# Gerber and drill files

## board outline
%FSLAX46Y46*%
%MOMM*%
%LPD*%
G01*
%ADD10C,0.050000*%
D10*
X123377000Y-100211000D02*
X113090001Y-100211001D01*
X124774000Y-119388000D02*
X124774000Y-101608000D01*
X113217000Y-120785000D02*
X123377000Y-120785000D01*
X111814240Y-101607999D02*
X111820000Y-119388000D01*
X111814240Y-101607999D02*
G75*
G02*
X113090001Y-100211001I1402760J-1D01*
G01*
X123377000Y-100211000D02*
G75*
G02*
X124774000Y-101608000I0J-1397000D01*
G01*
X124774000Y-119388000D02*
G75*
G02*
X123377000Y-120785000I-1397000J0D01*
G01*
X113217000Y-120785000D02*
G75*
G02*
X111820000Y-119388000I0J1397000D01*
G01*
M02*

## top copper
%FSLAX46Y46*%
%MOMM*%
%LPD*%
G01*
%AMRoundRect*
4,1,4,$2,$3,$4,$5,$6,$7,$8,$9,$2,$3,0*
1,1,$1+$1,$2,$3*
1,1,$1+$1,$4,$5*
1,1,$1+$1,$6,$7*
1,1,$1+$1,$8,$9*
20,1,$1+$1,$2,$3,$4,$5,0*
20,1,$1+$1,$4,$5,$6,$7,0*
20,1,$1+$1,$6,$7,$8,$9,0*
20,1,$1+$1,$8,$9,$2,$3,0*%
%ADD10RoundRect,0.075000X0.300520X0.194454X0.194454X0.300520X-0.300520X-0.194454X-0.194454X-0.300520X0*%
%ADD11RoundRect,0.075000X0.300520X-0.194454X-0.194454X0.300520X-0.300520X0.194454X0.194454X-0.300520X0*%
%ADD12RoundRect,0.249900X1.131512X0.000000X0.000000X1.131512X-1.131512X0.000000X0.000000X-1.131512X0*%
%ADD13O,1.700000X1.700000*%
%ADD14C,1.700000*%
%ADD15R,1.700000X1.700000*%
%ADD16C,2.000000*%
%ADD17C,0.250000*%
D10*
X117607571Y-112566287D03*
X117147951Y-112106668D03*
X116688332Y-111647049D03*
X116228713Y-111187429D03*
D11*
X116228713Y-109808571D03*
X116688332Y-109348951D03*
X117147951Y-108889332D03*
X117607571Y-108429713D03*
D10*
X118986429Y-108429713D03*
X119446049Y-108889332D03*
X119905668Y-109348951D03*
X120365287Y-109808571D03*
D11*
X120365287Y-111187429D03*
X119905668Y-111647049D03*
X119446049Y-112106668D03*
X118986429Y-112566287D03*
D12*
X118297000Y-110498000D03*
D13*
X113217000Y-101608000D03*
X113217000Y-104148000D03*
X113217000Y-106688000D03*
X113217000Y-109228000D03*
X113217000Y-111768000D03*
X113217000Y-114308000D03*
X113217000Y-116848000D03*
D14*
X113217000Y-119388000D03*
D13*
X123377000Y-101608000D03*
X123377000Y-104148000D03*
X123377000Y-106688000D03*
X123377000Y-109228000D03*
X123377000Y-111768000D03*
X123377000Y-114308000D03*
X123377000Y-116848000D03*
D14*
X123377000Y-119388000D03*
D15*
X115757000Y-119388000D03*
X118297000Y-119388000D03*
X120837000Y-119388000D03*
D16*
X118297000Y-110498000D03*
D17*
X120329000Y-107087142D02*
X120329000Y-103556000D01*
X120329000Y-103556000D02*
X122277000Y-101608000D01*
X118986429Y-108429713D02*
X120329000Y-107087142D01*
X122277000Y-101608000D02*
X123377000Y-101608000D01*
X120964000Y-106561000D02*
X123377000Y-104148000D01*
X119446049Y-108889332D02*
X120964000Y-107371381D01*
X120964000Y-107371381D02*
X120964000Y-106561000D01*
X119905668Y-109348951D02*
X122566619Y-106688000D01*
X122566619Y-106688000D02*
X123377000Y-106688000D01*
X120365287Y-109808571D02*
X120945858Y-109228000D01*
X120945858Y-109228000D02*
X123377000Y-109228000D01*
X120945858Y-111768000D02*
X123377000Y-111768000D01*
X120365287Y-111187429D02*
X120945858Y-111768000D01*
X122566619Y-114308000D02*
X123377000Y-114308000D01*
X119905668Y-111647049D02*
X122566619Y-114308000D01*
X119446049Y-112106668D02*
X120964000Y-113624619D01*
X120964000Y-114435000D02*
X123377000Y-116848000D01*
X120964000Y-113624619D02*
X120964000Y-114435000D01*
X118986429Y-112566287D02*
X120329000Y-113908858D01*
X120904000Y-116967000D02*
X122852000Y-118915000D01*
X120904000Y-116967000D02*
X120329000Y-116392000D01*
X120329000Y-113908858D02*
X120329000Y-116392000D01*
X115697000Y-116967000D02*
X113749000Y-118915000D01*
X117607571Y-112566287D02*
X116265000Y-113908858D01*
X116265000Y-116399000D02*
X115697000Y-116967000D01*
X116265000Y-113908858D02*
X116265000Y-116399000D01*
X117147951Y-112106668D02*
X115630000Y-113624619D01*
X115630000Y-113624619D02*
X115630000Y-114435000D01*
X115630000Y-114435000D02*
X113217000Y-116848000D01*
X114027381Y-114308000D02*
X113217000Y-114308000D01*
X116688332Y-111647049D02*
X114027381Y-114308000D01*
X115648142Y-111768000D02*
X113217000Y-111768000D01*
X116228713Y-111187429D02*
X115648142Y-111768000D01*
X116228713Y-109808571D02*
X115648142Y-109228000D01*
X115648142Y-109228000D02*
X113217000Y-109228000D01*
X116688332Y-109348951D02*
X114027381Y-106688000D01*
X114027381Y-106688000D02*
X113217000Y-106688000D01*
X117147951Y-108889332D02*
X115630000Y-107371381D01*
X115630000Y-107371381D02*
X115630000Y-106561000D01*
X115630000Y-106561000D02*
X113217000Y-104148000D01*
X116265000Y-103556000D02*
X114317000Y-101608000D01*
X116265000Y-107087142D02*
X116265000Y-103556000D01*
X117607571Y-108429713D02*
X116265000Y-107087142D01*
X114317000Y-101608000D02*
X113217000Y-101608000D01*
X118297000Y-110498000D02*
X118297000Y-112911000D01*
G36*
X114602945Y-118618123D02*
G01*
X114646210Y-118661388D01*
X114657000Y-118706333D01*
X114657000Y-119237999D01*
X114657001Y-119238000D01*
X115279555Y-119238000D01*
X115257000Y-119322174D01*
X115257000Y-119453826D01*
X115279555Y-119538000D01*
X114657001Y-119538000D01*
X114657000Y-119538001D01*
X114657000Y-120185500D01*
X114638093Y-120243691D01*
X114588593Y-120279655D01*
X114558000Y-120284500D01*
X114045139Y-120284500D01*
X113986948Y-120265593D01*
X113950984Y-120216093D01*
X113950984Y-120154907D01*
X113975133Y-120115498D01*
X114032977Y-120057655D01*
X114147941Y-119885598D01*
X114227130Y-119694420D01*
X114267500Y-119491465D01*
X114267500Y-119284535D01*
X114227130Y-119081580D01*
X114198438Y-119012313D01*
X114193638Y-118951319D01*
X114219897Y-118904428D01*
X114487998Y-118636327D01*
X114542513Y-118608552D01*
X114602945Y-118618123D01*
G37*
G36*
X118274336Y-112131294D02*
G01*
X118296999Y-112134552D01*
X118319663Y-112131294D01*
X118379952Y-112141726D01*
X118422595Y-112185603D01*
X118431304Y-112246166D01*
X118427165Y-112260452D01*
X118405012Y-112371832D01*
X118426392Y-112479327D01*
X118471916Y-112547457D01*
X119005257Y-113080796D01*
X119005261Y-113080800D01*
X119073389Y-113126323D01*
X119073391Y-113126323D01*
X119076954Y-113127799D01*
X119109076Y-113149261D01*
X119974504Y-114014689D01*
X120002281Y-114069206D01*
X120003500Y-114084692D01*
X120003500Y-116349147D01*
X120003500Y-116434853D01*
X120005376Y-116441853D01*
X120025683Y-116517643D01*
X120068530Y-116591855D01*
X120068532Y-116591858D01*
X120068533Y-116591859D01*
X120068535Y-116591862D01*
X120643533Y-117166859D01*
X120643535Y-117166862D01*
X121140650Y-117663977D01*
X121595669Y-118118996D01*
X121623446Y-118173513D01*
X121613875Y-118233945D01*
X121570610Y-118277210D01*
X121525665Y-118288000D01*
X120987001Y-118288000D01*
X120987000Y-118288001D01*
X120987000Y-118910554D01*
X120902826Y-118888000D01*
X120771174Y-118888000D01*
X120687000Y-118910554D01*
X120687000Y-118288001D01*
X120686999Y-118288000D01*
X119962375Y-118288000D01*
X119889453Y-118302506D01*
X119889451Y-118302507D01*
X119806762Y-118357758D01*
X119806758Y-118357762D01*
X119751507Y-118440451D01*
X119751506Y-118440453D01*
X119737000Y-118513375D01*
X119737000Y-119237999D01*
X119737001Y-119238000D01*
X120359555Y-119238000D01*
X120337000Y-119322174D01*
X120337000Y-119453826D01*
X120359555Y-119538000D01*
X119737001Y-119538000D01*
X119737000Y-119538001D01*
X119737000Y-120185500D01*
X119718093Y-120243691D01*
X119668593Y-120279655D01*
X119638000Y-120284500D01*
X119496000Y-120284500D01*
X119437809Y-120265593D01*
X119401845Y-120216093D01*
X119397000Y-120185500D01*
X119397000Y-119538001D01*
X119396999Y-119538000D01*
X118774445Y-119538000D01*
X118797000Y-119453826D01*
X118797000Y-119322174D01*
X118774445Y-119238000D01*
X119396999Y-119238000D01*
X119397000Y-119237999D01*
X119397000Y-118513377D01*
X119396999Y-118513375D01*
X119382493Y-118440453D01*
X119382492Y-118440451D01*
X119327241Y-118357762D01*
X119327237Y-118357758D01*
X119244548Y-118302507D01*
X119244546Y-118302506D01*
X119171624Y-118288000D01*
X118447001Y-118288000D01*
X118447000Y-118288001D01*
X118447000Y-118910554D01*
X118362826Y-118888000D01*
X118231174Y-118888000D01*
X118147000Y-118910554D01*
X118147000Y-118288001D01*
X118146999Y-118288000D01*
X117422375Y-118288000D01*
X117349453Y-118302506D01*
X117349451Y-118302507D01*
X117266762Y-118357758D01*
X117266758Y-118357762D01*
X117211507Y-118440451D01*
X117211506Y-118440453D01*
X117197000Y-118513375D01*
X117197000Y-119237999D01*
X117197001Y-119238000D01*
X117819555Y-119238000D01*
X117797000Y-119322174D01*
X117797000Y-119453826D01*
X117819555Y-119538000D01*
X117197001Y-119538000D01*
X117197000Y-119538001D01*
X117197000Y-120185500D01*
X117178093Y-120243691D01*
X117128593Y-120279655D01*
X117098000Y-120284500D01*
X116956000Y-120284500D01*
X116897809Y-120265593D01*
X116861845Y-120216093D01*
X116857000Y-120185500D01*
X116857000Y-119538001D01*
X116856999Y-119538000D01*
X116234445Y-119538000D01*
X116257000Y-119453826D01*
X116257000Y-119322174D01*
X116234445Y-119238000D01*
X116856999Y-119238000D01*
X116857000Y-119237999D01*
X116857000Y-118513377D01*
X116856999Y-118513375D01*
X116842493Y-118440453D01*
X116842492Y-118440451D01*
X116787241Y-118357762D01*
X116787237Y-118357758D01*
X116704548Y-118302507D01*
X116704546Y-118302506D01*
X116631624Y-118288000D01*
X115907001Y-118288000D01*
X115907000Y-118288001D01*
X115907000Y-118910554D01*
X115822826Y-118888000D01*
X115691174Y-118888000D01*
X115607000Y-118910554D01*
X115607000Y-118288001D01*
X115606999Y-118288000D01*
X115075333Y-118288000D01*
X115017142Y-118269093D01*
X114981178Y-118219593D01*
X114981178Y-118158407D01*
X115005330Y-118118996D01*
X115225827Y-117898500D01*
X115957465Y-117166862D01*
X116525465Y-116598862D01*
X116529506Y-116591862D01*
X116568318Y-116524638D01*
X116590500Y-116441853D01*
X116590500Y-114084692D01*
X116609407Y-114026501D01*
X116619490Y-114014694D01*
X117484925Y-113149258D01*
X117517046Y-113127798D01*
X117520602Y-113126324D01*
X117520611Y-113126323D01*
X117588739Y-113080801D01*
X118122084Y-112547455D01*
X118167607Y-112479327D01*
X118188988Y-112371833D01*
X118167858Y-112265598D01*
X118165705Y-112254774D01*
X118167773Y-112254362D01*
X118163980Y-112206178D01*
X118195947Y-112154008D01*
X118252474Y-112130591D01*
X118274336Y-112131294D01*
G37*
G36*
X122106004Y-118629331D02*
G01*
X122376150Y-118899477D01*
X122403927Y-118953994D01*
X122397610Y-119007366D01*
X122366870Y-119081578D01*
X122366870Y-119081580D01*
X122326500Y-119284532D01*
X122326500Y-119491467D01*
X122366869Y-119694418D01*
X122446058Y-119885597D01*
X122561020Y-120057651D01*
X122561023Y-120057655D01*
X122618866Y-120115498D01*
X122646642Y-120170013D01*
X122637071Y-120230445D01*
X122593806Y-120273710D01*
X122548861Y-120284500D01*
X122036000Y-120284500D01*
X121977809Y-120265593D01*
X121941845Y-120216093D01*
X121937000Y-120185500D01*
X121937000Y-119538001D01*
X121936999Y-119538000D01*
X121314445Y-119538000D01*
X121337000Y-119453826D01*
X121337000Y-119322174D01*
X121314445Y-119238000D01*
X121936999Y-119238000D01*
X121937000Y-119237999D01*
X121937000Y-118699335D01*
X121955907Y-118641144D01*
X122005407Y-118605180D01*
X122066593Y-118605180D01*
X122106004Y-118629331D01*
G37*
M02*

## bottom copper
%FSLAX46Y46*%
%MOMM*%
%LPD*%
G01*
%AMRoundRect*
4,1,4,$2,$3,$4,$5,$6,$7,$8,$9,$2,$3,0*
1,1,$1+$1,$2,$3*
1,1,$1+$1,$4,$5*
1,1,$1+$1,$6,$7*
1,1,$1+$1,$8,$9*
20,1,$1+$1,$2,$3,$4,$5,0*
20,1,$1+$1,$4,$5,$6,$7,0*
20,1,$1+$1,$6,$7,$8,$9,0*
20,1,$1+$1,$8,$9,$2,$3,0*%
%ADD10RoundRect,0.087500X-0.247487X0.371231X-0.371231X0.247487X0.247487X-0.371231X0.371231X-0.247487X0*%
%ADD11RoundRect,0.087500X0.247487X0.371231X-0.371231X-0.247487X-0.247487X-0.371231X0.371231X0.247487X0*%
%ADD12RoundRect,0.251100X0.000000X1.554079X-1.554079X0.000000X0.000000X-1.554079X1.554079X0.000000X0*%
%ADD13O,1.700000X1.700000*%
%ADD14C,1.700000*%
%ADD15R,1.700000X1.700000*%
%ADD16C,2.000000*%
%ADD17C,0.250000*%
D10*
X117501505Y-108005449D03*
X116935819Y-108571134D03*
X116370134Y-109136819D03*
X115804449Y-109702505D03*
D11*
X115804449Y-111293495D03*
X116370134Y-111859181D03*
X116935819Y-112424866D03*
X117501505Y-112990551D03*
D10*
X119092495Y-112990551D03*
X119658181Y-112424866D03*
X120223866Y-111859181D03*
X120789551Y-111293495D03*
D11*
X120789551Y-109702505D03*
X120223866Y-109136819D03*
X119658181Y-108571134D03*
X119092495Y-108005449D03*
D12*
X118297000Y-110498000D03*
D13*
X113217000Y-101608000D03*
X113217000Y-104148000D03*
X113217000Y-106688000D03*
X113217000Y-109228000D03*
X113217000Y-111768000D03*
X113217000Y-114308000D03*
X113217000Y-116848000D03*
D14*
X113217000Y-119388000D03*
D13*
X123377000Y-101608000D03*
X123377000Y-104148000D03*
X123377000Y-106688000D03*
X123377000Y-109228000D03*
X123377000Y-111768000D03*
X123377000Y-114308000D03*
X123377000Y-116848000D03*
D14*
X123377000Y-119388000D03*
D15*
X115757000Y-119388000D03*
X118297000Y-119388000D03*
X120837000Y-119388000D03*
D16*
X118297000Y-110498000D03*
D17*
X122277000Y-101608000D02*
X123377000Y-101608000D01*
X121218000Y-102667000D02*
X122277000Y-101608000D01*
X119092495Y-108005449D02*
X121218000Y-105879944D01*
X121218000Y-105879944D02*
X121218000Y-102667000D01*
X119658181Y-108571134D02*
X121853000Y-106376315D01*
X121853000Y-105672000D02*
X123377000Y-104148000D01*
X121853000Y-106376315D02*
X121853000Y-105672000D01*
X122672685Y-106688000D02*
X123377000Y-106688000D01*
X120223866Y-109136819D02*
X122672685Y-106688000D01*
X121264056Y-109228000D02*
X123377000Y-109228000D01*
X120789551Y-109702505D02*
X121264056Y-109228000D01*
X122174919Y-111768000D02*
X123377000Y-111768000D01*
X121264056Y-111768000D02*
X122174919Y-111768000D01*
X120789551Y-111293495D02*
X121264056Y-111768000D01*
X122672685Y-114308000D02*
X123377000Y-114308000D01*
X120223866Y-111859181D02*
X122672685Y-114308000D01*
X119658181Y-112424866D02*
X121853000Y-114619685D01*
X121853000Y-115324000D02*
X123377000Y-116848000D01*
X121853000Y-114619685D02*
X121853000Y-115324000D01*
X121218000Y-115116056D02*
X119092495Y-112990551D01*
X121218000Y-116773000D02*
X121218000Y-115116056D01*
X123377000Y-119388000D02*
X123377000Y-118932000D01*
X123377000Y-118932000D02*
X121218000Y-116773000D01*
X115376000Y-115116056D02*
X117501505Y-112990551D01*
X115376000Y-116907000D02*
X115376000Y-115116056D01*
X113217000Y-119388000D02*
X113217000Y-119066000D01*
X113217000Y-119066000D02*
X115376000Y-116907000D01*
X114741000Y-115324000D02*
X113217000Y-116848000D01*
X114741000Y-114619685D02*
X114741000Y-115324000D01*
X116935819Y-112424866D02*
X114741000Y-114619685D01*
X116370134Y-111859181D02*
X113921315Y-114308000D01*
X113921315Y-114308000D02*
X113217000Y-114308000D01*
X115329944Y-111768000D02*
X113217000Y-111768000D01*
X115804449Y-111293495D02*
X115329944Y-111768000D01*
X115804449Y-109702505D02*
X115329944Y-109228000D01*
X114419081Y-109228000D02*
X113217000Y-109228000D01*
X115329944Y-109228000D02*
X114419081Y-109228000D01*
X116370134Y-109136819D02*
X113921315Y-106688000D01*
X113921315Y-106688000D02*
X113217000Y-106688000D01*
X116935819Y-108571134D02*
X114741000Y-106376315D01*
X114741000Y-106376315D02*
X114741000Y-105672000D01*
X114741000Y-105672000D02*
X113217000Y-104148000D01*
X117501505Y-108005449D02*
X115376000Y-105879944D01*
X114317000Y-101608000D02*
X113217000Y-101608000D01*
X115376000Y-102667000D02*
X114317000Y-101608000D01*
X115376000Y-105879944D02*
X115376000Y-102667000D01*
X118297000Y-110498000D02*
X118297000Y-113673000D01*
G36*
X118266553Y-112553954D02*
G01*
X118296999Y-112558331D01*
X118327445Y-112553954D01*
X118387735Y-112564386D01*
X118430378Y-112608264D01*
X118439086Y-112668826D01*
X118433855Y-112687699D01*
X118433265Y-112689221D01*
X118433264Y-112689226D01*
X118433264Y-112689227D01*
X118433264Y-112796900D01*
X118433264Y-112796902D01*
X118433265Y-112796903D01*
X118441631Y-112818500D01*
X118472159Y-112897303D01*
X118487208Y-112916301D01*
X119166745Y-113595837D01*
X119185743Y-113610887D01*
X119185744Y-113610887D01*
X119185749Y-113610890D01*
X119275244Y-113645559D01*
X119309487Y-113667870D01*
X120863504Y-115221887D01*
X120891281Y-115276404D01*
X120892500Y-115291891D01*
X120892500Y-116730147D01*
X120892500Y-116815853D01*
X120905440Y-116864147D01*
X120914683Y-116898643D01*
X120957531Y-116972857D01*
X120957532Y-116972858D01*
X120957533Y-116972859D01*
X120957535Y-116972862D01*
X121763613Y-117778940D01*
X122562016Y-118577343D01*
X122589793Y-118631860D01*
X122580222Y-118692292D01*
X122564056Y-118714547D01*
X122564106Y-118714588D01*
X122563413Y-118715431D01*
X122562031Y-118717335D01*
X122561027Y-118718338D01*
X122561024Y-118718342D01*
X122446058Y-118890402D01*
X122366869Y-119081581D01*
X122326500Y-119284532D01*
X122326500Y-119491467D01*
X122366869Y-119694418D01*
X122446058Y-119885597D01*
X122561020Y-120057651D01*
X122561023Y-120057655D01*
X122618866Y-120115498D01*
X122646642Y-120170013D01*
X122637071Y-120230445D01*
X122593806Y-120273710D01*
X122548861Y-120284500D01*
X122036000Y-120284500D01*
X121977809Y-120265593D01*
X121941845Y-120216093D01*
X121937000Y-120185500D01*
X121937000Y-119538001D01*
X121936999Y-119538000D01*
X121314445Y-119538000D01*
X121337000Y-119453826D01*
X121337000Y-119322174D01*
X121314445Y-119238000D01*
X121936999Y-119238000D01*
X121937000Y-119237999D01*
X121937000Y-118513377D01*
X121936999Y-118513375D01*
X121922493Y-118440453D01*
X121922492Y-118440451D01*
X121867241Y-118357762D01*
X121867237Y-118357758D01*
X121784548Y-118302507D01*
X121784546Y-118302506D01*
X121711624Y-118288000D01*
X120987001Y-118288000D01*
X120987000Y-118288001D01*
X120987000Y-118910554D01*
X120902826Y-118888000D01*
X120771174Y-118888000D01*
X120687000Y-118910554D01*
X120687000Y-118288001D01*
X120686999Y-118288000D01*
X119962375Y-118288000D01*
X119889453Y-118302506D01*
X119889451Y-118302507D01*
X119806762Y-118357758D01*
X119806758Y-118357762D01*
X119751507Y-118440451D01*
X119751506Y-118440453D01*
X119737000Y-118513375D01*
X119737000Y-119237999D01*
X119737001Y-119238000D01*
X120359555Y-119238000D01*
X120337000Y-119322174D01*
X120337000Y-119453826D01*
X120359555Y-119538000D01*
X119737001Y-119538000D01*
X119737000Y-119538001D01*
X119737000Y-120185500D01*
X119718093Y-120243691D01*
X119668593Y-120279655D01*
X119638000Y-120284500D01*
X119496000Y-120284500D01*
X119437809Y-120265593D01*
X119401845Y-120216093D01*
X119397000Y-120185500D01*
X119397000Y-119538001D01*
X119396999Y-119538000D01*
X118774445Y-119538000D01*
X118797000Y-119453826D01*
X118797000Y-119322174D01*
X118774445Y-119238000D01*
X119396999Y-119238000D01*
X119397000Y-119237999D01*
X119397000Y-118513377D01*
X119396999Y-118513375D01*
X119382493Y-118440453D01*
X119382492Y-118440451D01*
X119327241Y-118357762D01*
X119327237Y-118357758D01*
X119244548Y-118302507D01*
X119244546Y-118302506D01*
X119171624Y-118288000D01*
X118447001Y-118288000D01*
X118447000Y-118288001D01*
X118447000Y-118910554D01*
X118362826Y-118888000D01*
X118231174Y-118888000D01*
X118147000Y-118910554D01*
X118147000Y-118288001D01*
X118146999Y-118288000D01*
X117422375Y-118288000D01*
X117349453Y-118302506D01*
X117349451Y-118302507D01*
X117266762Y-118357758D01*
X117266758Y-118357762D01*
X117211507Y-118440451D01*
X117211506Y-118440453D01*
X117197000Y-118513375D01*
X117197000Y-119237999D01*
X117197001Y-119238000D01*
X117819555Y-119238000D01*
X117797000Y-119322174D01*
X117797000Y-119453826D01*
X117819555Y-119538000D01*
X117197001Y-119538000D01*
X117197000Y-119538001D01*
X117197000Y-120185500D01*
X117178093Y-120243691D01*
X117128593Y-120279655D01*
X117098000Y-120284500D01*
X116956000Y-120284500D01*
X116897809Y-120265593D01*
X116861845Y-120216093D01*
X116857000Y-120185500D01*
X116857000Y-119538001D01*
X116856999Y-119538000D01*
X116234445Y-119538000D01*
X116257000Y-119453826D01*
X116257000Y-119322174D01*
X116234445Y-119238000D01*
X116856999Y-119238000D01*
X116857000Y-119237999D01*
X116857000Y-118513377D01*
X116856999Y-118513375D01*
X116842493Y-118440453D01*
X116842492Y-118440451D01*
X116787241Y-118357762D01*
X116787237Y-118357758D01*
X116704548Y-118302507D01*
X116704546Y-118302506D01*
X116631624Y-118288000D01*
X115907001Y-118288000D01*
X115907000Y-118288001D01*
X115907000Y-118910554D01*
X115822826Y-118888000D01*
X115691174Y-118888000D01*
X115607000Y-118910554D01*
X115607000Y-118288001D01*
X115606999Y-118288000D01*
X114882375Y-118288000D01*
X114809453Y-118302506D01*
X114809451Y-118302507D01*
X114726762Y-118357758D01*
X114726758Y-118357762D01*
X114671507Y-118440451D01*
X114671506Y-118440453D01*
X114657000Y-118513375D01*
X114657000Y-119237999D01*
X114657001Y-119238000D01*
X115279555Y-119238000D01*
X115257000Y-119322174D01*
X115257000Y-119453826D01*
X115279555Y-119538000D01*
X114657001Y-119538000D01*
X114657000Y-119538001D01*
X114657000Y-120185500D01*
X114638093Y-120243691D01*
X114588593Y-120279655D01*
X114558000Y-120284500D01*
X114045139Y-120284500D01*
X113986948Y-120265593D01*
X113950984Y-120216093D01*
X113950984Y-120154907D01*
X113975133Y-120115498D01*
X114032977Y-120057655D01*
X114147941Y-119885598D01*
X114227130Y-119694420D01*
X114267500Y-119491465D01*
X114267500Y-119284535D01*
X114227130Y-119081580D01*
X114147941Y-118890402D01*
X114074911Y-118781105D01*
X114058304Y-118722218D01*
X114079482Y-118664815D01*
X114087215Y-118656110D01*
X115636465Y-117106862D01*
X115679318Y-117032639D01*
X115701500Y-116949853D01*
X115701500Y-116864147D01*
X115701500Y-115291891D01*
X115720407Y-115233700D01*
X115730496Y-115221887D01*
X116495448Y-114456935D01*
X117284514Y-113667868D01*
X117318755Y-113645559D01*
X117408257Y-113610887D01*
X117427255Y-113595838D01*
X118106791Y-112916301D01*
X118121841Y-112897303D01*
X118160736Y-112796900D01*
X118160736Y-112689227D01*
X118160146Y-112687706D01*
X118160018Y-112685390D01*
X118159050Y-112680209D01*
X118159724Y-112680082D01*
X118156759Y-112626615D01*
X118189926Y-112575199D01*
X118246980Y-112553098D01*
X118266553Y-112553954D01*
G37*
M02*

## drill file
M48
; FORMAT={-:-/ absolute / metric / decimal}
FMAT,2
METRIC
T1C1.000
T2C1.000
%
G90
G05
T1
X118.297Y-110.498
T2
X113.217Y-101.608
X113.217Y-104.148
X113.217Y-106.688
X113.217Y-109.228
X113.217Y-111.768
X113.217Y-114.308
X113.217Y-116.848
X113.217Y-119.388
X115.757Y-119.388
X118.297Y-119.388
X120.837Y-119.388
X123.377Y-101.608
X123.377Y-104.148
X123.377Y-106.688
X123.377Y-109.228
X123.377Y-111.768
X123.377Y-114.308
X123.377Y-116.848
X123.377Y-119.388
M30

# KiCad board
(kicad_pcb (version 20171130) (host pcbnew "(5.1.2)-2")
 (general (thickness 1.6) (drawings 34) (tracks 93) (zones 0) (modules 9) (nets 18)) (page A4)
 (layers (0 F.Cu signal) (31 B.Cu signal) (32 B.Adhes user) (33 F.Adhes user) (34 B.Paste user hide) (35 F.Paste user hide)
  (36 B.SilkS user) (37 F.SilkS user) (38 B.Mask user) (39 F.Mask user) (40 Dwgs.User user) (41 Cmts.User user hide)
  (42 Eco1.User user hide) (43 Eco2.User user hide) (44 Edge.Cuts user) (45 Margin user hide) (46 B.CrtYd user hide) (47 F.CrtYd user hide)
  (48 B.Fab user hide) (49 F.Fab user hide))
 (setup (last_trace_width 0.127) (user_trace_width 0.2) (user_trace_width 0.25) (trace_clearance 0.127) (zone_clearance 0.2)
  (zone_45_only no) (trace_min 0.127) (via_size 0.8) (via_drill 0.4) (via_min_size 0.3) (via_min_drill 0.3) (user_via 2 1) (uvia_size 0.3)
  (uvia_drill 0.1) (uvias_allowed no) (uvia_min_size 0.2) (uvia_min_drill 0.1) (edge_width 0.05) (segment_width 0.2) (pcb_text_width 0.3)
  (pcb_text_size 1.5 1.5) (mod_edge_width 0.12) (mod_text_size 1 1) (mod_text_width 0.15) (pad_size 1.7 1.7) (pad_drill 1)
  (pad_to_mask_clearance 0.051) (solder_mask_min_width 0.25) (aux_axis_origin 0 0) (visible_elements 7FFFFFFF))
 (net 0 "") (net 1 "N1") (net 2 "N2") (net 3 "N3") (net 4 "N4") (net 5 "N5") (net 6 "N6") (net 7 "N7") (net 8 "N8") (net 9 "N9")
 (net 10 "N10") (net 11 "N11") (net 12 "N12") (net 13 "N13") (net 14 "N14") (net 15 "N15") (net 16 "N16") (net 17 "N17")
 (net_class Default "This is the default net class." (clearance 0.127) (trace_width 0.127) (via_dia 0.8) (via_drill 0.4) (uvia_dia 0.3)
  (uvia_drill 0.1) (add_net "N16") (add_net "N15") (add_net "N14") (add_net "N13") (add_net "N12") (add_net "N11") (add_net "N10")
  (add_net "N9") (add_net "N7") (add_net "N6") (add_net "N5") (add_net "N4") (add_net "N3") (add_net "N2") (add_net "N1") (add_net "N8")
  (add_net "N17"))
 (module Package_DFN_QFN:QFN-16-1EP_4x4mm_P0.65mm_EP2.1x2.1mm (layer F.Cu) (at 118.297 110.498 135)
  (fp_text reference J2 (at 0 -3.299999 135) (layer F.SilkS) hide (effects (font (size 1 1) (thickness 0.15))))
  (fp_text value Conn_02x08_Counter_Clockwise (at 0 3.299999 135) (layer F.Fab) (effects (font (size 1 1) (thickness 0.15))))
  (pad 16 smd roundrect (at -0.975 -1.95 135) (size 0.3 0.85) (layers F.Cu F.Paste F.Mask) (roundrect_rratio 0.25) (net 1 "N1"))
  (pad 15 smd roundrect (at -0.325 -1.95 135) (size 0.3 0.85) (layers F.Cu F.Paste F.Mask) (roundrect_rratio 0.25) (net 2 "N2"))
  (pad 14 smd roundrect (at 0.325 -1.95 135) (size 0.3 0.85) (layers F.Cu F.Paste F.Mask) (roundrect_rratio 0.25) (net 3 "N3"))
  (pad 13 smd roundrect (at 0.975 -1.95 135) (size 0.3 0.85) (layers F.Cu F.Paste F.Mask) (roundrect_rratio 0.25) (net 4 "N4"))
  (pad 12 smd roundrect (at 1.95 -0.975 135) (size 0.85 0.3) (layers F.Cu F.Paste F.Mask) (roundrect_rratio 0.25) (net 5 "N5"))
  (pad 11 smd roundrect (at 1.95 -0.325 135) (size 0.85 0.3) (layers F.Cu F.Paste F.Mask) (roundrect_rratio 0.25) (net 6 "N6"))
  (pad 10 smd roundrect (at 1.95 0.325 135) (size 0.85 0.3) (layers F.Cu F.Paste F.Mask) (roundrect_rratio 0.25) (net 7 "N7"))
  (pad 9 smd roundrect (at 1.95 0.975 135) (size 0.85 0.3) (layers F.Cu F.Paste F.Mask) (roundrect_rratio 0.25) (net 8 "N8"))
  (pad 8 smd roundrect (at 0.975 1.95 135) (size 0.3 0.85) (layers F.Cu F.Paste F.Mask) (roundrect_rratio 0.25) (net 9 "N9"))
  (pad 7 smd roundrect (at 0.325 1.95 135) (size 0.3 0.85) (layers F.Cu F.Paste F.Mask) (roundrect_rratio 0.25) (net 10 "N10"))
  (pad 6 smd roundrect (at -0.325 1.95 135) (size 0.3 0.85) (layers F.Cu F.Paste F.Mask) (roundrect_rratio 0.25) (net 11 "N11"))
  (pad 5 smd roundrect (at -0.975 1.95 135) (size 0.3 0.85) (layers F.Cu F.Paste F.Mask) (roundrect_rratio 0.25) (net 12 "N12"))
  (pad 4 smd roundrect (at -1.95 0.975 135) (size 0.85 0.3) (layers F.Cu F.Paste F.Mask) (roundrect_rratio 0.25) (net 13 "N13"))
  (pad 3 smd roundrect (at -1.95 0.325 135) (size 0.85 0.3) (layers F.Cu F.Paste F.Mask) (roundrect_rratio 0.25) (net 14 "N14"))
  (pad 2 smd roundrect (at -1.95 -0.325 135) (size 0.85 0.3) (layers F.Cu F.Paste F.Mask) (roundrect_rratio 0.25) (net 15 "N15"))
  (pad 1 smd roundrect (at -1.95 -0.975 135) (size 0.85 0.3) (layers F.Cu F.Paste F.Mask) (roundrect_rratio 0.25) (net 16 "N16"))
  (pad "" smd roundrect (at 0.525 0.525 135) (size 0.85 0.85) (layers F.Paste) (roundrect_rratio 0.25))
  (pad "" smd roundrect (at 0.525 -0.525 135) (size 0.85 0.85) (layers F.Paste) (roundrect_rratio 0.25))
  (pad "" smd roundrect (at -0.525 0.525 135) (size 0.85 0.85) (layers F.Paste) (roundrect_rratio 0.25))
  (pad "" smd roundrect (at -0.525 -0.525 135) (size 0.85 0.85) (layers F.Paste) (roundrect_rratio 0.25))
  (pad 17 smd roundrect (at 0 0 135) (size 2.1 2.1) (layers F.Cu F.Mask) (roundrect_rratio 0.119) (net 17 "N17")))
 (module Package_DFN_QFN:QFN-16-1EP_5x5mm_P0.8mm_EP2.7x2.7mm (layer B.Cu) (at 118.297 110.498 225)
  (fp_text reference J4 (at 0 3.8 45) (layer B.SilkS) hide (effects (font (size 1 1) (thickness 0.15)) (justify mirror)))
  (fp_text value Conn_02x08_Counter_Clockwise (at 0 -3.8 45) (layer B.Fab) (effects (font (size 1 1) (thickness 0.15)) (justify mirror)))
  (pad 16 smd roundrect (at -1.2 2.325 225) (size 0.35 1.05) (layers B.Cu B.Paste B.Mask) (roundrect_rratio 0.25) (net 8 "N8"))
  (pad 15 smd roundrect (at -0.4 2.325 225) (size 0.35 1.05) (layers B.Cu B.Paste B.Mask) (roundrect_rratio 0.25) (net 7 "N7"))
  (pad 14 smd roundrect (at 0.4 2.325 225) (size 0.35 1.05) (layers B.Cu B.Paste B.Mask) (roundrect_rratio 0.25) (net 6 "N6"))
  (pad 13 smd roundrect (at 1.2 2.325 225) (size 0.35 1.05) (layers B.Cu B.Paste B.Mask) (roundrect_rratio 0.25) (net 5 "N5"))
  (pad 12 smd roundrect (at 2.325 1.2 225) (size 1.05 0.35) (layers B.Cu B.Paste B.Mask) (roundrect_rratio 0.25) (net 4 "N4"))
  (pad 11 smd roundrect (at 2.325 0.4 225) (size 1.05 0.35) (layers B.Cu B.Paste B.Mask) (roundrect_rratio 0.25) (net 3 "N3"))
  (pad 10 smd roundrect (at 2.325 -0.4 225) (size 1.05 0.35) (layers B.Cu B.Paste B.Mask) (roundrect_rratio 0.25) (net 2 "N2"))
  (pad 9 smd roundrect (at 2.325 -1.2 225) (size 1.05 0.35) (layers B.Cu B.Paste B.Mask) (roundrect_rratio 0.25) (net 1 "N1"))
  (pad 8 smd roundrect (at 1.2 -2.325 225) (size 0.35 1.05) (layers B.Cu B.Paste B.Mask) (roundrect_rratio 0.25) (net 16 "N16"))
  (pad 7 smd roundrect (at 0.4 -2.325 225) (size 0.35 1.05) (layers B.Cu B.Paste B.Mask) (roundrect_rratio 0.25) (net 15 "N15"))
  (pad 6 smd roundrect (at -0.4 -2.325 225) (size 0.35 1.05) (layers B.Cu B.Paste B.Mask) (roundrect_rratio 0.25) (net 14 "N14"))
  (pad 5 smd roundrect (at -1.2 -2.325 225) (size 0.35 1.05) (layers B.Cu B.Paste B.Mask) (roundrect_rratio 0.25) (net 13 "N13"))
  (pad 4 smd roundrect (at -2.325 -1.2 225) (size 1.05 0.35) (layers B.Cu B.Paste B.Mask) (roundrect_rratio 0.25) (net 12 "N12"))
  (pad 3 smd roundrect (at -2.325 -0.4 225) (size 1.05 0.35) (layers B.Cu B.Paste B.Mask) (roundrect_rratio 0.25) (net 11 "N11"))
  (pad 2 smd roundrect (at -2.325 0.4 225) (size 1.05 0.35) (layers B.Cu B.Paste B.Mask) (roundrect_rratio 0.25) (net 10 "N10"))
  (pad 1 smd roundrect (at -2.325 1.2 225) (size 1.05 0.35) (layers B.Cu B.Paste B.Mask) (roundrect_rratio 0.25) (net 9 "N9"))
  (pad "" smd roundrect (at 0.675 -0.675 225) (size 1.09 1.09) (layers B.Paste) (roundrect_rratio 0.229358))
  (pad "" smd roundrect (at 0.675 0.675 225) (size 1.09 1.09) (layers B.Paste) (roundrect_rratio 0.229358))
  (pad "" smd roundrect (at -0.675 -0.675 225) (size 1.09 1.09) (layers B.Paste) (roundrect_rratio 0.229358))
  (pad "" smd roundrect (at -0.675 0.675 225) (size 1.09 1.09) (layers B.Paste) (roundrect_rratio 0.229358))
  (pad 17 smd roundrect (at 0 0 225) (size 2.7 2.7) (layers B.Cu B.Mask) (roundrect_rratio 0.09300000000000001) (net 17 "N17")))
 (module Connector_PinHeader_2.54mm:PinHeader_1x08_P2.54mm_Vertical (layer B.Cu) (at 113.217 119.388)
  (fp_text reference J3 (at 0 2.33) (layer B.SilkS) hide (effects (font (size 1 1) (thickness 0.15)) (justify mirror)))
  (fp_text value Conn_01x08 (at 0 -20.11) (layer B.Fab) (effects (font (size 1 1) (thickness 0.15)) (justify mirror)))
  (pad 8 thru_hole oval (at 0 -17.78) (size 1.7 1.7) (drill 1) (layers *.Cu *.Mask) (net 8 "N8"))
  (pad 7 thru_hole oval (at 0 -15.24) (size 1.7 1.7) (drill 1) (layers *.Cu *.Mask) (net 7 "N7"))
  (pad 6 thru_hole oval (at 0 -12.7) (size 1.7 1.7) (drill 1) (layers *.Cu *.Mask) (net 6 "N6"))
  (pad 5 thru_hole oval (at 0 -10.16) (size 1.7 1.7) (drill 1) (layers *.Cu *.Mask) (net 5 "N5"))
  (pad 4 thru_hole oval (at 0 -7.62) (size 1.7 1.7) (drill 1) (layers *.Cu *.Mask) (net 4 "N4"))
  (pad 3 thru_hole oval (at 0 -5.08) (size 1.7 1.7) (drill 1) (layers *.Cu *.Mask) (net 3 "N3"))
  (pad 2 thru_hole oval (at 0 -2.54) (size 1.7 1.7) (drill 1) (layers *.Cu *.Mask) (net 2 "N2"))
  (pad 1 thru_hole circle (at 0 0) (size 1.7 1.7) (drill 1) (layers *.Cu *.Mask) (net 1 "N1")))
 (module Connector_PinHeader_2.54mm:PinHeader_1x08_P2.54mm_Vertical (layer B.Cu) (at 123.377 119.388)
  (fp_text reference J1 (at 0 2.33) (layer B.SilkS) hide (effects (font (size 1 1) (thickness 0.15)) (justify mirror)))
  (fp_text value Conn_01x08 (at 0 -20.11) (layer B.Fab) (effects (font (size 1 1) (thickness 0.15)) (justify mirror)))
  (pad 8 thru_hole oval (at 0 -17.78) (size 1.7 1.7) (drill 1) (layers *.Cu *.Mask) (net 9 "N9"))
  (pad 7 thru_hole oval (at 0 -15.24) (size 1.7 1.7) (drill 1) (layers *.Cu *.Mask) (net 10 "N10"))
  (pad 6 thru_hole oval (at 0 -12.7) (size 1.7 1.7) (drill 1) (layers *.Cu *.Mask) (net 11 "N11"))
  (pad 5 thru_hole oval (at 0 -10.16) (size 1.7 1.7) (drill 1) (layers *.Cu *.Mask) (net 12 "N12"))
  (pad 4 thru_hole oval (at 0 -7.62) (size 1.7 1.7) (drill 1) (layers *.Cu *.Mask) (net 13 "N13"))
  (pad 3 thru_hole oval (at 0 -5.08) (size 1.7 1.7) (drill 1) (layers *.Cu *.Mask) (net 14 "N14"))
  (pad 2 thru_hole oval (at 0 -2.54) (size 1.7 1.7) (drill 1) (layers *.Cu *.Mask) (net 15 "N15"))
  (pad 1 thru_hole circle (at 0 0) (size 1.7 1.7) (drill 1) (layers *.Cu *.Mask) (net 16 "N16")))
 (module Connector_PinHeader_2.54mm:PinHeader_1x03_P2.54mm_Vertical (layer B.Cu) (at 120.837 119.388 90)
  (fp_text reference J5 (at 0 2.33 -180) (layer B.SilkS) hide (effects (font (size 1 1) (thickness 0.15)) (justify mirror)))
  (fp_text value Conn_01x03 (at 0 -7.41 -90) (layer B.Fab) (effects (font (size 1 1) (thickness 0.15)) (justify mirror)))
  (pad 3 thru_hole rect (at 0 -5.08 90) (size 1.7 1.7) (drill 1) (layers *.Cu *.Mask) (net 17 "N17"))
  (pad 2 thru_hole rect (at 0 -2.54 90) (size 1.7 1.7) (drill 1) (layers *.Cu *.Mask) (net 17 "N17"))
  (pad 1 thru_hole rect (at 0 0 90) (size 1.7 1.7) (drill 1) (layers *.Cu *.Mask) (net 17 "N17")))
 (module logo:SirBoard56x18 (layer B.Cu) (at 118.297 105.672 180)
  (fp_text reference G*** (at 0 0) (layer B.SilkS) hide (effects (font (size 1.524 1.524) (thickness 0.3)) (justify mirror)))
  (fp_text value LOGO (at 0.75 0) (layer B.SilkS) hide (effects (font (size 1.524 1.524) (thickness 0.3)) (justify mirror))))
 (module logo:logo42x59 (layer B.Cu) (at 118.297 102.497 180)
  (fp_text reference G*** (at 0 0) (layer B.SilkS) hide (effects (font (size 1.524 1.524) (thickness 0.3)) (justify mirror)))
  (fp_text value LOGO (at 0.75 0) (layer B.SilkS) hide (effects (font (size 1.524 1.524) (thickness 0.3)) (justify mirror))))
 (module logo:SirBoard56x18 (layer F.Cu) (at 118.301 106.175)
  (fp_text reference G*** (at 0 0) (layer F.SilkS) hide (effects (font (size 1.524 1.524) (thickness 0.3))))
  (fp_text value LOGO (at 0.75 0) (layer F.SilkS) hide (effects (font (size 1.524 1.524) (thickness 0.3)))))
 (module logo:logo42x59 (layer F.Cu) (at 118.301 102.775)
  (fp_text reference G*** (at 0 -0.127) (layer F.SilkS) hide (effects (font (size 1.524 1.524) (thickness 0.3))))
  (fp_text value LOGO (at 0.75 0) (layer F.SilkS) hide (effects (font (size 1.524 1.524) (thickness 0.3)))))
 (gr_line (start 123.377 100.211) (end 113.090001 100.211001) (layer Edge.Cuts) (width 0.05))
 (gr_line (start 124.774 119.388) (end 124.774 101.608) (layer Edge.Cuts) (width 0.05))
 (gr_line (start 113.217 120.785) (end 123.377 120.785) (layer Edge.Cuts) (width 0.05))
 (gr_line (start 111.81424 101.607999) (end 111.82 119.388) (layer Edge.Cuts) (width 0.05))
 (gr_arc (start 113.217 101.608) (end 113.090001 100.211001) (angle -84.80557109) (layer Edge.Cuts) (width 0.05))
 (gr_arc (start 123.377 101.608) (end 124.774 101.608) (angle -90) (layer Edge.Cuts) (width 0.05))
 (gr_arc (start 123.377 119.388) (end 123.377 120.785) (angle -90) (layer Edge.Cuts) (width 0.05))
 (gr_arc (start 113.217 119.388) (end 111.82 119.388) (angle -90) (layer Edge.Cuts) (width 0.05))
 (segment (start 120.329 107.087142) (end 120.329 103.556) (width 0.25) (layer F.Cu) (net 9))
 (segment (start 120.329 103.556) (end 122.277 101.608) (width 0.25) (layer F.Cu) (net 9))
 (segment (start 118.986429 108.429713) (end 120.329 107.087142) (width 0.25) (layer F.Cu) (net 9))
 (segment (start 122.277 101.608) (end 123.377 101.608) (width 0.25) (layer F.Cu) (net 9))
 (segment (start 122.277 101.608) (end 123.377 101.608) (width 0.25) (layer B.Cu) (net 9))
 (segment (start 121.218 102.667) (end 122.277 101.608) (width 0.25) (layer B.Cu) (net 9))
 (segment (start 119.092495 108.005449) (end 121.218 105.879944) (width 0.25) (layer B.Cu) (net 9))
 (segment (start 121.218 105.879944) (end 121.218 102.667) (width 0.25) (layer B.Cu) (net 9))
 (segment (start 119.658181 108.571134) (end 121.853 106.376315) (width 0.25) (layer B.Cu) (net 10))
 (segment (start 121.853 105.672) (end 123.377 104.148) (width 0.25) (layer B.Cu) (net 10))
 (segment (start 121.853 106.376315) (end 121.853 105.672) (width 0.25) (layer B.Cu) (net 10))
 (segment (start 120.964 106.561) (end 123.377 104.148) (width 0.25) (layer F.Cu) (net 10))
 (segment (start 119.446049 108.889332) (end 120.964 107.371381) (width 0.25) (layer F.Cu) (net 10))
 (segment (start 120.964 107.371381) (end 120.964 106.561) (width 0.25) (layer F.Cu) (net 10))
 (segment (start 122.672685 106.688) (end 123.377 106.688) (width 0.25) (layer B.Cu) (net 11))
 (segment (start 120.223866 109.136819) (end 122.672685 106.688) (width 0.25) (layer B.Cu) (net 11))
 (segment (start 119.905668 109.348951) (end 122.566619 106.688) (width 0.25) (layer F.Cu) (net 11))
 (segment (start 122.566619 106.688) (end 123.377 106.688) (width 0.25) (layer F.Cu) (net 11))
 (segment (start 120.365287 109.808571) (end 120.945858 109.228) (width 0.25) (layer F.Cu) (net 12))
 (segment (start 120.945858 109.228) (end 123.377 109.228) (width 0.25) (layer F.Cu) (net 12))
 (segment (start 121.264056 109.228) (end 123.377 109.228) (width 0.25) (layer B.Cu) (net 12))
 (segment (start 120.789551 109.702505) (end 121.264056 109.228) (width 0.25) (layer B.Cu) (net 12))
 (segment (start 120.945858 111.768) (end 123.377 111.768) (width 0.25) (layer F.Cu) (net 13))
 (segment (start 120.365287 111.187429) (end 120.945858 111.768) (width 0.25) (layer F.Cu) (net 13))
 (segment (start 122.174919 111.768) (end 123.377 111.768) (width 0.25) (layer B.Cu) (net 13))
 (segment (start 121.264056 111.768) (end 122.174919 111.768) (width 0.25) (layer B.Cu) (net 13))
 (segment (start 120.789551 111.293495) (end 121.264056 111.768) (width 0.25) (layer B.Cu) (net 13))
 (segment (start 122.566619 114.308) (end 123.377 114.308) (width 0.25) (layer F.Cu) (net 14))
 (segment (start 119.905668 111.647049) (end 122.566619 114.308) (width 0.25) (layer F.Cu) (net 14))
 (segment (start 122.672685 114.308) (end 123.377 114.308) (width 0.25) (layer B.Cu) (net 14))
 (segment (start 120.223866 111.859181) (end 122.672685 114.308) (width 0.25) (layer B.Cu) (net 14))
 (segment (start 119.446049 112.106668) (end 120.964 113.624619) (width 0.25) (layer F.Cu) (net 15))
 (segment (start 120.964 114.435) (end 123.377 116.848) (width 0.25) (layer F.Cu) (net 15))
 (segment (start 120.964 113.624619) (end 120.964 114.435) (width 0.25) (layer F.Cu) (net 15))
 (segment (start 119.658181 112.424866) (end 121.853 114.619685) (width 0.25) (layer B.Cu) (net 15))
 (segment (start 121.853 115.324) (end 123.377 116.848) (width 0.25) (layer B.Cu) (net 15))
 (segment (start 121.853 114.619685) (end 121.853 115.324) (width 0.25) (layer B.Cu) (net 15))
 (segment (start 118.986429 112.566287) (end 120.329 113.908858) (width 0.25) (layer F.Cu) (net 16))
 (segment (start 120.904 116.967) (end 122.852 118.915) (width 0.25) (layer F.Cu) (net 16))
 (segment (start 121.218 115.116056) (end 119.092495 112.990551) (width 0.25) (layer B.Cu) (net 16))
 (segment (start 121.218 116.773) (end 121.218 115.116056) (width 0.25) (layer B.Cu) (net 16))
 (segment (start 123.377 119.388) (end 123.377 118.932) (width 0.25) (layer B.Cu) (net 16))
 (segment (start 123.377 118.932) (end 121.218 116.773) (width 0.25) (layer B.Cu) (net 16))
 (segment (start 120.904 116.967) (end 120.329 116.392) (width 0.25) (layer F.Cu) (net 16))
 (segment (start 120.329 113.908858) (end 120.329 116.392) (width 0.25) (layer F.Cu) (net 16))
 (segment (start 115.376 115.116056) (end 117.501505 112.990551) (width 0.25) (layer B.Cu) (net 1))
 (segment (start 115.376 116.907) (end 115.376 115.116056) (width 0.25) (layer B.Cu) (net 1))
 (segment (start 113.217 119.388) (end 113.217 119.066) (width 0.25) (layer B.Cu) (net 1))
 (segment (start 113.217 119.066) (end 115.376 116.907) (width 0.25) (layer B.Cu) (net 1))
 (segment (start 115.697 116.967) (end 113.749 118.915) (width 0.25) (layer F.Cu) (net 1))
 (segment (start 117.607571 112.566287) (end 116.265 113.908858) (width 0.25) (layer F.Cu) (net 1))
 (segment (start 116.265 116.399) (end 115.697 116.967) (width 0.25) (layer F.Cu) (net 1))
 (segment (start 116.265 113.908858) (end 116.265 116.399) (width 0.25) (layer F.Cu) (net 1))
 (segment (start 114.741 115.324) (end 113.217 116.848) (width 0.25) (layer B.Cu) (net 2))
 (segment (start 114.741 114.619685) (end 114.741 115.324) (width 0.25) (layer B.Cu) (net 2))
 (segment (start 116.935819 112.424866) (end 114.741 114.619685) (width 0.25) (layer B.Cu) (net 2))
 (segment (start 117.147951 112.106668) (end 115.63 113.624619) (width 0.25) (layer F.Cu) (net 2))
 (segment (start 115.63 113.624619) (end 115.63 114.435) (width 0.25) (layer F.Cu) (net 2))
 (segment (start 115.63 114.435) (end 113.217 116.848) (width 0.25) (layer F.Cu) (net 2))
 (segment (start 116.370134 111.859181) (end 113.921315 114.308) (width 0.25) (layer B.Cu) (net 3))
 (segment (start 113.921315 114.308) (end 113.217 114.308) (width 0.25) (layer B.Cu) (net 3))
 (segment (start 114.027381 114.308) (end 113.217 114.308) (width 0.25) (layer F.Cu) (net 3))
 (segment (start 116.688332 111.647049) (end 114.027381 114.308) (width 0.25) (layer F.Cu) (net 3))
 (segment (start 115.648142 111.768) (end 113.217 111.768) (width 0.25) (layer F.Cu) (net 4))
 (segment (start 116.228713 111.187429) (end 115.648142 111.768) (width 0.25) (layer F.Cu) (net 4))
 (segment (start 115.329944 111.768) (end 113.217 111.768) (width 0.25) (layer B.Cu) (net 4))
 (segment (start 115.804449 111.293495) (end 115.329944 111.768) (width 0.25) (layer B.Cu) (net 4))
 (segment (start 115.804449 109.702505) (end 115.329944 109.228) (width 0.25) (layer B.Cu) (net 5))
 (segment (start 114.419081 109.228) (end 113.217 109.228) (width 0.25) (layer B.Cu) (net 5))
 (segment (start 115.329944 109.228) (end 114.419081 109.228) (width 0.25) (layer B.Cu) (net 5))
 (segment (start 116.228713 109.808571) (end 115.648142 109.228) (width 0.25) (layer F.Cu) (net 5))
 (segment (start 115.648142 109.228) (end 113.217 109.228) (width 0.25) (layer F.Cu) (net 5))
 (segment (start 116.370134 109.136819) (end 113.921315 106.688) (width 0.25) (layer B.Cu) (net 6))
 (segment (start 113.921315 106.688) (end 113.217 106.688) (width 0.25) (layer B.Cu) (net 6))
 (segment (start 116.688332 109.348951) (end 114.027381 106.688) (width 0.25) (layer F.Cu) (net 6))
 (segment (start 114.027381 106.688) (end 113.217 106.688) (width 0.25) (layer F.Cu) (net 6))
 (segment (start 116.935819 108.571134) (end 114.741 106.376315) (width 0.25) (layer B.Cu) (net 7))
 (segment (start 114.741 106.376315) (end 114.741 105.672) (width 0.25) (layer B.Cu) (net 7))
 (segment (start 114.741 105.672) (end 113.217 104.148) (width 0.25) (layer B.Cu) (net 7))
 (segment (start 117.147951 108.889332) (end 115.63 107.371381) (width 0.25) (layer F.Cu) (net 7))
 (segment (start 115.63 107.371381) (end 115.63 106.561) (width 0.25) (layer F.Cu) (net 7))
 (segment (start 115.63 106.561) (end 113.217 104.148) (width 0.25) (layer F.Cu) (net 7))
 (segment (start 117.501505 108.005449) (end 115.376 105.879944) (width 0.25) (layer B.Cu) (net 8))
 (segment (start 114.317 101.608) (end 113.217 101.608) (width 0.25) (layer B.Cu) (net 8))
 (segment (start 115.376 102.667) (end 114.317 101.608) (width 0.25) (layer B.Cu) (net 8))
 (segment (start 115.376 105.879944) (end 115.376 102.667) (width 0.25) (layer B.Cu) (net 8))
 (segment (start 116.265 103.556) (end 114.317 101.608) (width 0.25) (layer F.Cu) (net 8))
 (segment (start 116.265 107.087142) (end 116.265 103.556) (width 0.25) (layer F.Cu) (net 8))
 (segment (start 117.607571 108.429713) (end 116.265 107.087142) (width 0.25) (layer F.Cu) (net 8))
 (segment (start 114.317 101.608) (end 113.217 101.608) (width 0.25) (layer F.Cu) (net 8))
 (via (at 118.297 110.498) (size 2) (drill 1) (layers F.Cu B.Cu) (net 17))
 (segment (start 118.297 110.498) (end 118.297 113.673) (width 0.25) (layer B.Cu) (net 17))
 (segment (start 118.297 110.498) (end 118.297 112.911) (width 0.25) (layer F.Cu) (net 17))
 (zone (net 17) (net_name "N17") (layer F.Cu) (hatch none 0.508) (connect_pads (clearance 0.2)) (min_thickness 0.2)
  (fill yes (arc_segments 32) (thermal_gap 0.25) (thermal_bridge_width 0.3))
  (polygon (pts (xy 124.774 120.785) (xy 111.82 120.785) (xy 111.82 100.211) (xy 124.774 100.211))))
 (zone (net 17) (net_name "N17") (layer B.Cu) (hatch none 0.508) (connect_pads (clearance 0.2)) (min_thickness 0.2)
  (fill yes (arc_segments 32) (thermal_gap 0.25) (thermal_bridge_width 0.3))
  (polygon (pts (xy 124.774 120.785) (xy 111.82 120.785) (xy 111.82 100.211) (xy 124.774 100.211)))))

